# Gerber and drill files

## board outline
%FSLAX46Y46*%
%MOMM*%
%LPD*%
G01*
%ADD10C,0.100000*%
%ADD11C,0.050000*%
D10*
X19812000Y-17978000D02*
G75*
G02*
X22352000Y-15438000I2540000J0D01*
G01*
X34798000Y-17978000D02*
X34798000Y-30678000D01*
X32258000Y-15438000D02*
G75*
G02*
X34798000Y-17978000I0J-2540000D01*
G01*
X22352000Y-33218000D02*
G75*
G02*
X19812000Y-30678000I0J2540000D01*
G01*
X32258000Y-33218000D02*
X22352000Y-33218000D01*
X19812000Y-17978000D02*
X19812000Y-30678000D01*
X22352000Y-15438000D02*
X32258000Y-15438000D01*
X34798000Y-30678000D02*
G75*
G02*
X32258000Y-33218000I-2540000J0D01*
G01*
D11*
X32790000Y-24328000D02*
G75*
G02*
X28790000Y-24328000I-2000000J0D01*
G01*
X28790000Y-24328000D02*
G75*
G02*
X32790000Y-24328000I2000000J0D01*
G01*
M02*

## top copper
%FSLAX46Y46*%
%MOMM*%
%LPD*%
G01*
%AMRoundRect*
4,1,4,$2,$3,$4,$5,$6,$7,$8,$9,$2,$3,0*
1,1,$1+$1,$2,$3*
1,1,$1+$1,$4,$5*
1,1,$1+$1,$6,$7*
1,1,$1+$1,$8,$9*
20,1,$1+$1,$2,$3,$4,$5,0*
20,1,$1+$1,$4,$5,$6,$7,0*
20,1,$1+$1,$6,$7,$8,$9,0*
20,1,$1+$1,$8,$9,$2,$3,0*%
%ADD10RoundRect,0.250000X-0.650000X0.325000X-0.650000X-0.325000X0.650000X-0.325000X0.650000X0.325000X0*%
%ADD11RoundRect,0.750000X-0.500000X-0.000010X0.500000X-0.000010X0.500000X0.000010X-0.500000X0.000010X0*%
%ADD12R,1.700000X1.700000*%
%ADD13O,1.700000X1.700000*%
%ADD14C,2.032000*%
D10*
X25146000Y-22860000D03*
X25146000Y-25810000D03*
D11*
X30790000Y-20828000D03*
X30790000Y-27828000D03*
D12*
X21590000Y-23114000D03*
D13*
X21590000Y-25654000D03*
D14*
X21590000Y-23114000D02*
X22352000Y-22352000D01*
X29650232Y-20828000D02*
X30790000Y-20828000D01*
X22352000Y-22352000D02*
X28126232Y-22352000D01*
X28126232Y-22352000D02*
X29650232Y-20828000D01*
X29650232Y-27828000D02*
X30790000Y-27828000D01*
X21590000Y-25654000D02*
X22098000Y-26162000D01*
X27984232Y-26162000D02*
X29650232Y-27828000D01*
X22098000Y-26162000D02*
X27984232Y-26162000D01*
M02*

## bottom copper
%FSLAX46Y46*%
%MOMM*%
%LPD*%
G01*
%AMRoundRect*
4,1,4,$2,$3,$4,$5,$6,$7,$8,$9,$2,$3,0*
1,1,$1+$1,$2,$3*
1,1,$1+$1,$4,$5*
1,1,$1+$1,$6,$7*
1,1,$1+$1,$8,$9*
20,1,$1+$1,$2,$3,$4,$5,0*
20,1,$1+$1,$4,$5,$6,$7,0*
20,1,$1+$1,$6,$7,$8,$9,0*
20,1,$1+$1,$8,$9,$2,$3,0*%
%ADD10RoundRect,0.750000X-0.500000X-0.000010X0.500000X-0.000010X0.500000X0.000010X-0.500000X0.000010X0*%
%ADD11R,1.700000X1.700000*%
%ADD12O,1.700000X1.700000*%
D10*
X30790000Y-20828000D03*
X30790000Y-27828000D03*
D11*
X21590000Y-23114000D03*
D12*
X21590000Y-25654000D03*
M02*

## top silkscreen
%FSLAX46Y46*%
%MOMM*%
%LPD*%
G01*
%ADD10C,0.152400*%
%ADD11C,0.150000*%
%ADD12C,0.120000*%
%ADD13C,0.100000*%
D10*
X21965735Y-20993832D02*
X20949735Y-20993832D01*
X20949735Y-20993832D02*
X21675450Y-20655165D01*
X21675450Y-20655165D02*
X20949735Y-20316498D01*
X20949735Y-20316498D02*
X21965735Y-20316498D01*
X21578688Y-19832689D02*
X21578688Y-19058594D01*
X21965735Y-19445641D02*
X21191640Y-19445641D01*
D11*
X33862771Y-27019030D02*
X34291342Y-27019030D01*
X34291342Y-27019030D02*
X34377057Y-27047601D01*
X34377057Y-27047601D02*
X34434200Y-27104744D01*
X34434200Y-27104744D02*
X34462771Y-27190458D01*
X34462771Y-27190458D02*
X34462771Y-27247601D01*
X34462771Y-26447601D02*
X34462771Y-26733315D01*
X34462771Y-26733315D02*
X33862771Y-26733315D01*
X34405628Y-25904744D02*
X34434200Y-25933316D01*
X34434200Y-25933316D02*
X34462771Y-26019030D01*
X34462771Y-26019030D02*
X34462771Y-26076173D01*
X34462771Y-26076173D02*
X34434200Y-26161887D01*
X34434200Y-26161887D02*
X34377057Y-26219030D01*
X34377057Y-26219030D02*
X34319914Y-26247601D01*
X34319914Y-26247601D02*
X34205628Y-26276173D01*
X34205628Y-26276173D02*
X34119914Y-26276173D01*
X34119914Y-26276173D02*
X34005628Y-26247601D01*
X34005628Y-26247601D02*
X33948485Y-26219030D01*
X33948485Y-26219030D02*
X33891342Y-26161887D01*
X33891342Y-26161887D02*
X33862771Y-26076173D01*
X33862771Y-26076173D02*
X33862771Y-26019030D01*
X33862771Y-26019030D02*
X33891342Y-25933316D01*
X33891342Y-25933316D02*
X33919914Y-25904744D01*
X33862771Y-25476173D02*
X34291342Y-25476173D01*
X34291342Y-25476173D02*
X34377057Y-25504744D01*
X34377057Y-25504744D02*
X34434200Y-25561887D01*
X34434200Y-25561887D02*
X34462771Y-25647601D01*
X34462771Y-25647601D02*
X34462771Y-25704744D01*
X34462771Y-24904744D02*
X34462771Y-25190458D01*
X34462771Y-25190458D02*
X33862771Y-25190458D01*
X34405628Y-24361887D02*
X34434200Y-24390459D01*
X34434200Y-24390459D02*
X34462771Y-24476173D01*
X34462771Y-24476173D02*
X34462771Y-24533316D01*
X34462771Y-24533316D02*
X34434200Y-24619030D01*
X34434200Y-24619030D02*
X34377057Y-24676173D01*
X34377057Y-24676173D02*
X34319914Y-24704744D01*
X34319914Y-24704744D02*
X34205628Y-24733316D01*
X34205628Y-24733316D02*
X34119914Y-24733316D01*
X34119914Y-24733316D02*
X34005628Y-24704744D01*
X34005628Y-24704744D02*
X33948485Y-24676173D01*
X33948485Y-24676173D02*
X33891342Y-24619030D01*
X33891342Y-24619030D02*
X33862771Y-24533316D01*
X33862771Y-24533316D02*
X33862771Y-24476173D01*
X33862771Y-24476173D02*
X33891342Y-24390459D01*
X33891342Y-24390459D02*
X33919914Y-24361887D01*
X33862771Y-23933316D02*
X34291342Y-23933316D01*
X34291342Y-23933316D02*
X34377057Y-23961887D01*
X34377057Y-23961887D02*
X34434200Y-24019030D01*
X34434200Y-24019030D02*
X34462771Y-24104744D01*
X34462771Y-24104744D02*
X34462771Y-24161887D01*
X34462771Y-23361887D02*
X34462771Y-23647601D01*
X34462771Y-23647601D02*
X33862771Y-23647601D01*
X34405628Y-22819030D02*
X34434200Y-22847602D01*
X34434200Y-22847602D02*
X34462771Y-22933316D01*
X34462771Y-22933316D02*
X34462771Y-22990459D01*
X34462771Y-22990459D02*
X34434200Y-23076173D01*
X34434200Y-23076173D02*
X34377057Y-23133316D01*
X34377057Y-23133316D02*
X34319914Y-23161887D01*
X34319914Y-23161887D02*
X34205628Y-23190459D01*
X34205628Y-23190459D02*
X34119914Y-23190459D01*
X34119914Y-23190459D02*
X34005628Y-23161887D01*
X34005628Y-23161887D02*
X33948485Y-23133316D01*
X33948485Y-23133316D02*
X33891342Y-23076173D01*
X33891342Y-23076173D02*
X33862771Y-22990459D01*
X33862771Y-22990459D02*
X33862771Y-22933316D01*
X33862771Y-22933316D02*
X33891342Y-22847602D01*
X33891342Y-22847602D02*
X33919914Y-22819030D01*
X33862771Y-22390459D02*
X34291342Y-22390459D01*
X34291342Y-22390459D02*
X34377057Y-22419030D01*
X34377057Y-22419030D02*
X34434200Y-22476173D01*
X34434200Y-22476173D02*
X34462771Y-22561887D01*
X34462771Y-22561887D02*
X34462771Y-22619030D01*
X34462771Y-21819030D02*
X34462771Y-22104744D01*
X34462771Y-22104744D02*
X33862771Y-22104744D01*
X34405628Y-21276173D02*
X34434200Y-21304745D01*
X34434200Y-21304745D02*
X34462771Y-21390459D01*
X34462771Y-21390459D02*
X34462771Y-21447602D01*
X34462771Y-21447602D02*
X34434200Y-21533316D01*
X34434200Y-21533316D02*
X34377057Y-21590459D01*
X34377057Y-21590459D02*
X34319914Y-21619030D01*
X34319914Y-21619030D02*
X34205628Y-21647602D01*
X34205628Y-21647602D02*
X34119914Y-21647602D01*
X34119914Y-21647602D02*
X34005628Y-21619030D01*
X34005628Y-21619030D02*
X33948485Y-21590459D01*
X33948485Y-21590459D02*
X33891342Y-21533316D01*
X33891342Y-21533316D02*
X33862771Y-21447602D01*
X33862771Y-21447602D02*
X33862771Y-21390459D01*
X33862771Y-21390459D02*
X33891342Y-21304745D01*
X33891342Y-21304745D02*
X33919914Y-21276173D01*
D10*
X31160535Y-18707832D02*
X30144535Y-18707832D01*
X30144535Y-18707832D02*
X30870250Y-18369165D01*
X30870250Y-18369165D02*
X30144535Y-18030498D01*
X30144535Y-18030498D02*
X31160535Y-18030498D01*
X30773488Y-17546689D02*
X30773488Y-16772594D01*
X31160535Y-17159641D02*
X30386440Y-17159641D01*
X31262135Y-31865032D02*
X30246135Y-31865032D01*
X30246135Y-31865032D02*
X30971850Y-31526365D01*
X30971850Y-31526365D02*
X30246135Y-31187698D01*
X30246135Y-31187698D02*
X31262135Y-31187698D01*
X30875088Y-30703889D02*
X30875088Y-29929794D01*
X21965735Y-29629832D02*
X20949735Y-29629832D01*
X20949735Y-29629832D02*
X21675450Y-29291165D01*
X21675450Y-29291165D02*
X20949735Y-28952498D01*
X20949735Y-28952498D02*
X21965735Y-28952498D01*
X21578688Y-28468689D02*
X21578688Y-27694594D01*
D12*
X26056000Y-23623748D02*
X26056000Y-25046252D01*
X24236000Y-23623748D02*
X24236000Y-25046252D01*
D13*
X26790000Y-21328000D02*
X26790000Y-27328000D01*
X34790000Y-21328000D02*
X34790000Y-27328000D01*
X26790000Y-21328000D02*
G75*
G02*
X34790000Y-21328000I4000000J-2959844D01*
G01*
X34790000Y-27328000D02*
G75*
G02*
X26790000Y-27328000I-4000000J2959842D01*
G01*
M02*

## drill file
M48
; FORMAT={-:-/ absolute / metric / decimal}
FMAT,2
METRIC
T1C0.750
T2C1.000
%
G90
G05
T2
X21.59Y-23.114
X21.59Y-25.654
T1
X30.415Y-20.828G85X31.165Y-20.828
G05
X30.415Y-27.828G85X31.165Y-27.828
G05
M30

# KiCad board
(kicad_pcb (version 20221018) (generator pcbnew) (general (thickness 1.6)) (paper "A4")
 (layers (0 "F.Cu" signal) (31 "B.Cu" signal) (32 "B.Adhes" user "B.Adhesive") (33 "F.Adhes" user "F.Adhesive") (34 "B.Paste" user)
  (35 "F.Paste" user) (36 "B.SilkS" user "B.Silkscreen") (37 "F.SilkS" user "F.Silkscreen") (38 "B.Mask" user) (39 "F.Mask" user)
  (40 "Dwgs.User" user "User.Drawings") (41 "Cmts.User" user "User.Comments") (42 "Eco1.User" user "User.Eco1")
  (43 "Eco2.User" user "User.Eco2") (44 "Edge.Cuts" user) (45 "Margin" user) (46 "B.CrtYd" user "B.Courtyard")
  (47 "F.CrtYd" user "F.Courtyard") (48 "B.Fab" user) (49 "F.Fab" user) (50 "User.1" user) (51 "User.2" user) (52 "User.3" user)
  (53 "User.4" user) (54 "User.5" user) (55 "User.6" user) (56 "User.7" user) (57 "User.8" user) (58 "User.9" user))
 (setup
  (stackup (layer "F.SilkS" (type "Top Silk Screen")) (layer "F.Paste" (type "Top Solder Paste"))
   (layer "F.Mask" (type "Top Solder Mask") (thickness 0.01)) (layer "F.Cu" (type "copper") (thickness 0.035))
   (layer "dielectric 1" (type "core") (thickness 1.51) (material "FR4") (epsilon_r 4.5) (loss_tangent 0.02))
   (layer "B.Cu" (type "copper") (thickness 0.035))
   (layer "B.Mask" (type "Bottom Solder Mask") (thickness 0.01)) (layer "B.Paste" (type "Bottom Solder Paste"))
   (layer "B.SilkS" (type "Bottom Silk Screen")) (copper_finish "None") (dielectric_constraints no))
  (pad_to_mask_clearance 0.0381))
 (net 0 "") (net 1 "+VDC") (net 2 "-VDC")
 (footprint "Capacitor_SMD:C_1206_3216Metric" (layer "F.Cu") (at 25.146 24.335 -90)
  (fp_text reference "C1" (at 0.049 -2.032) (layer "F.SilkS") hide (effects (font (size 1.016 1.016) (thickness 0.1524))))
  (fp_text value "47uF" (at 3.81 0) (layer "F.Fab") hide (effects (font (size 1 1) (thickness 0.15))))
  (fp_line (start -0.711252 -0.91) (end 0.711252 -0.91) (stroke (width 0.12) (type solid)) (layer "F.SilkS"))
  (fp_line (start -0.711252 0.91) (end 0.711252 0.91) (stroke (width 0.12) (type solid)) (layer "F.SilkS"))
  (pad "1" smd roundrect (at -1.475 0 270) (size 1.15 1.8) (layers "F.Cu" "F.Paste" "F.Mask") (roundrect_rratio 0.2173913043) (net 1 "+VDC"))
  (pad "2" smd roundrect (at 1.475 0 270) (size 1.15 1.8) (layers "F.Cu" "F.Paste" "F.Mask") (roundrect_rratio 0.2173913043) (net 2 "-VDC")))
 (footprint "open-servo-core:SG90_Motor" (layer "F.Cu") (at 30.79 24.328)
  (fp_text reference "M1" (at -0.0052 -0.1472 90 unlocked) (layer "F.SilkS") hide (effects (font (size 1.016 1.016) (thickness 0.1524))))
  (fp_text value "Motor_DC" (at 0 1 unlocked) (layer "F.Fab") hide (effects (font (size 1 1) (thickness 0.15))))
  (fp_line (start -4 -3) (end -4 3) (stroke (width 0.1) (type default)) (layer "F.SilkS"))
  (fp_line (start 4 -3) (end 4 3) (stroke (width 0.1) (type default)) (layer "F.SilkS"))
  (fp_arc (start -4 -3) (mid 0 -5.016166) (end 4 -3) (stroke (width 0.1) (type default)) (layer "F.SilkS"))
  (fp_arc (start 4 3) (mid 0 5.016167) (end -4 3) (stroke (width 0.1) (type default)) (layer "F.SilkS"))
  (fp_circle (center 0 0) (end 2 0) (stroke (width 0.05) (type default)) (fill none) (layer "Edge.Cuts"))
  (pad "1" thru_hole roundrect (at 0 -3.5) (size 2.5 1.5) (drill oval 1.5 0.75) (layers "*.Cu" "*.Mask") (roundrect_rratio 0.5)
   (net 1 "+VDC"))
  (pad "2" thru_hole roundrect (at 0 3.5) (size 2.5 1.5) (drill oval 1.5 0.75) (layers "*.Cu" "*.Mask") (roundrect_rratio 0.5)
   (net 2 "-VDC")))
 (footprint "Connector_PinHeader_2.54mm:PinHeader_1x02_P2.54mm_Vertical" (layer "B.Cu") (at 21.59 23.114 180)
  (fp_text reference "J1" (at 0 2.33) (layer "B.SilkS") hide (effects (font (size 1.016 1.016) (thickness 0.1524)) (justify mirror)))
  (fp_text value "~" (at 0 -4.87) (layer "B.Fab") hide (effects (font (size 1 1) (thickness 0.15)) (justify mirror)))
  (pad "1" thru_hole rect (at 0 0 180) (size 1.7 1.7) (drill 1) (layers "*.Cu" "*.Mask") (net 1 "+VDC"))
  (pad "2" thru_hole oval (at 0 -2.54 180) (size 1.7 1.7) (drill 1) (layers "*.Cu" "*.Mask") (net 2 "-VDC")))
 (gr_arc (start 19.812 17.978) (mid 20.555949 16.181949) (end 22.352 15.438) (stroke (width 0.1) (type default)) (layer "Edge.Cuts"))
 (gr_line (start 34.798 17.978) (end 34.798 30.678) (stroke (width 0.1) (type default)) (layer "Edge.Cuts"))
 (gr_arc (start 32.258 15.438) (mid 34.054051 16.181949) (end 34.798 17.978) (stroke (width 0.1) (type default)) (layer "Edge.Cuts"))
 (gr_arc (start 22.352 33.218) (mid 20.555949 32.474051) (end 19.812 30.678) (stroke (width 0.1) (type default)) (layer "Edge.Cuts"))
 (gr_line (start 32.258 33.218) (end 22.352 33.218) (stroke (width 0.1) (type default)) (layer "Edge.Cuts"))
 (gr_line (start 19.812 17.978) (end 19.812 30.678) (stroke (width 0.1) (type default)) (layer "Edge.Cuts"))
 (gr_line (start 22.352 15.438) (end 32.258 15.438) (stroke (width 0.1) (type default)) (layer "Edge.Cuts"))
 (gr_arc (start 34.798 30.678) (mid 34.054051 32.474051) (end 32.258 33.218) (stroke (width 0.1) (type default)) (layer "Edge.Cuts"))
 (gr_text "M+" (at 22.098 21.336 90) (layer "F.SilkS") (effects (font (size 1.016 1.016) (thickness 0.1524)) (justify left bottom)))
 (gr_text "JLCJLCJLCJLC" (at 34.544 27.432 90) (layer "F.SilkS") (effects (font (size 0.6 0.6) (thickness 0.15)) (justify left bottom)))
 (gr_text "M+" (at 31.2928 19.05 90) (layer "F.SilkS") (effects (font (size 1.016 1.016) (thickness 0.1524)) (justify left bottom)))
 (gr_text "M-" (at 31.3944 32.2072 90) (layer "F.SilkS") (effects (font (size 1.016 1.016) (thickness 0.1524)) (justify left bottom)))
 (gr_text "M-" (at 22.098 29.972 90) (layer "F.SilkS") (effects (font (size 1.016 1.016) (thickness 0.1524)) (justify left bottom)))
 (segment (start 21.59 23.114) (end 22.352 22.352) (width 2.032) (layer "F.Cu") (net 1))
 (segment (start 29.650232 20.828) (end 30.79 20.828) (width 2.032) (layer "F.Cu") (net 1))
 (segment (start 22.352 22.352) (end 28.126232 22.352) (width 2.032) (layer "F.Cu") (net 1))
 (segment (start 28.126232 22.352) (end 29.650232 20.828) (width 2.032) (layer "F.Cu") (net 1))
 (segment (start 29.650232 27.828) (end 30.79 27.828) (width 2.032) (layer "F.Cu") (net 2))
 (segment (start 21.59 25.654) (end 22.098 26.162) (width 2.032) (layer "F.Cu") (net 2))
 (segment (start 27.984232 26.162) (end 29.650232 27.828) (width 2.032) (layer "F.Cu") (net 2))
 (segment (start 22.098 26.162) (end 27.984232 26.162) (width 2.032) (layer "F.Cu") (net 2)))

